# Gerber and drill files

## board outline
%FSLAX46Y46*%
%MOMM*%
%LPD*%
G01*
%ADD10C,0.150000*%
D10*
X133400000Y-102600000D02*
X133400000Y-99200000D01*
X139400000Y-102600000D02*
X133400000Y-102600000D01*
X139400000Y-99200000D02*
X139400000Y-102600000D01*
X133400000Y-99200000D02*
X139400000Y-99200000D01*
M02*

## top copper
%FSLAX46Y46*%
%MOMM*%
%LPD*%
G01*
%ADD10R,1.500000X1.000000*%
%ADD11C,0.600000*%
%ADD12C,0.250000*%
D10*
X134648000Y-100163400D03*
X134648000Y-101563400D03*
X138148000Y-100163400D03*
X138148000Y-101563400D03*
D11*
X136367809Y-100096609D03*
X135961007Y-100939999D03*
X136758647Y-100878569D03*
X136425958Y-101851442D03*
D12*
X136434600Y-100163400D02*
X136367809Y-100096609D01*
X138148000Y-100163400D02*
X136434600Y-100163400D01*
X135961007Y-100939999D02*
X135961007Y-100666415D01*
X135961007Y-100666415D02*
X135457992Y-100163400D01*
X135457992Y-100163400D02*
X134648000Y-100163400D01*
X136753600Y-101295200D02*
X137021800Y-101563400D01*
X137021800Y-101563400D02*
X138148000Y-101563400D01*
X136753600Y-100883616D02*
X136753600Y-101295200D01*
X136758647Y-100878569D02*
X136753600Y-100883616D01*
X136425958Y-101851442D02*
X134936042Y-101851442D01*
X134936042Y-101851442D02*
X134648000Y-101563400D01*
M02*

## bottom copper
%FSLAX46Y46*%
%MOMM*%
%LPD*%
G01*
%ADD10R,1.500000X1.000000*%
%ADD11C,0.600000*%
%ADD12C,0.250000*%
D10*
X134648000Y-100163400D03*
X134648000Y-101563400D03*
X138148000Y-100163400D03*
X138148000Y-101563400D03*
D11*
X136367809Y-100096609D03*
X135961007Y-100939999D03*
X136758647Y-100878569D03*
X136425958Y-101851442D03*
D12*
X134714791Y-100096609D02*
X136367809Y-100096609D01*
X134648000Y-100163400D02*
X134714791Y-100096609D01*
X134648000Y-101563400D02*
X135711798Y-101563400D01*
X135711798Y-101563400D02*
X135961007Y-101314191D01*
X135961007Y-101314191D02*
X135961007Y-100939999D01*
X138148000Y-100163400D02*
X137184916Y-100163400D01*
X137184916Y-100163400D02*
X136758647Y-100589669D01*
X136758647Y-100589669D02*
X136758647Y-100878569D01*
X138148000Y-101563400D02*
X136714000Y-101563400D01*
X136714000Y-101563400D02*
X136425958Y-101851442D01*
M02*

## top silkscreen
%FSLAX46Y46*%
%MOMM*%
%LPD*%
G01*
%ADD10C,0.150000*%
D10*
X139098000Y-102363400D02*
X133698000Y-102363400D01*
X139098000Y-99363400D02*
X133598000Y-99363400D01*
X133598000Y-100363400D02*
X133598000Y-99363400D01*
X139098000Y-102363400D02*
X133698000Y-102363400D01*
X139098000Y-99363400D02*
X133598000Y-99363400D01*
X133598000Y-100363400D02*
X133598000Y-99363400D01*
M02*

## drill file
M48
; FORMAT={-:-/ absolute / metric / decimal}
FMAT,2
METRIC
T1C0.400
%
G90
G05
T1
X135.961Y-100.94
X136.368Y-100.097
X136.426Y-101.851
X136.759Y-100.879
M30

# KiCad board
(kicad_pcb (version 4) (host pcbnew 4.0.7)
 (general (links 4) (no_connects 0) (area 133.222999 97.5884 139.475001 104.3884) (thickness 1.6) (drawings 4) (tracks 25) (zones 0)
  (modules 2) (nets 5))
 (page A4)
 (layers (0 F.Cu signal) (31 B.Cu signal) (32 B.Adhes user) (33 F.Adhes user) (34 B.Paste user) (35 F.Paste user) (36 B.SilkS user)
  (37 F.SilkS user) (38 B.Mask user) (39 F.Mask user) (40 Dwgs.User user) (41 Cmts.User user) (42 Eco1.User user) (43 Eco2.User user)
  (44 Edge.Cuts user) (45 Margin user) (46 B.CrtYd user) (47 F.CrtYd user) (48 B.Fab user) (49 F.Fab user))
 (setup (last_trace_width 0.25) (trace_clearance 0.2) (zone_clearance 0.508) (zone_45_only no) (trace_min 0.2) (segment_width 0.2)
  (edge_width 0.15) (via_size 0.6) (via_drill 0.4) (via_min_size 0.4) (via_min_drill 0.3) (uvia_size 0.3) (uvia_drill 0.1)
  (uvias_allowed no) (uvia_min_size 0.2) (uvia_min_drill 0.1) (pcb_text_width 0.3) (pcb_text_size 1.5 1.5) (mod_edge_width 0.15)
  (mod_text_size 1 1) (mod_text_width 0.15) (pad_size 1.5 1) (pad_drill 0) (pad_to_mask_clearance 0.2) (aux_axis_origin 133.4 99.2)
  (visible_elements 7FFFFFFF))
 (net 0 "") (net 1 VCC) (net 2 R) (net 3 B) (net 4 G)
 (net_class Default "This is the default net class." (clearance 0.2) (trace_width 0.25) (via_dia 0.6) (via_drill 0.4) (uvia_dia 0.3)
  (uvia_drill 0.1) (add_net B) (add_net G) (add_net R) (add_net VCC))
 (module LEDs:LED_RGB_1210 (layer F.Cu) (at 136.398 100.8634)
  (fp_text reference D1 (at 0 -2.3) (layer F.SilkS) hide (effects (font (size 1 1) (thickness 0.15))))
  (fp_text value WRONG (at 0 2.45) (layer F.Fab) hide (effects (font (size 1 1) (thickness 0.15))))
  (fp_line (start 2.7 1.5) (end -2.7 1.5) (layer F.SilkS) (width 0.15))
  (fp_line (start 2.7 -1.5) (end -2.8 -1.5) (layer F.SilkS) (width 0.15))
  (fp_line (start -2.8 -0.5) (end -2.8 -1.5) (layer F.SilkS) (width 0.15))
  (pad 1 smd rect (at -1.75 -0.7 180) (size 1.5 1) (layers B.Cu B.Paste B.Mask) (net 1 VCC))
  (pad 2 smd rect (at -1.75 0.7 180) (size 1.5 1) (layers B.Cu B.Paste B.Mask) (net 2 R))
  (pad 4 smd rect (at 1.75 -0.7 180) (size 1.5 1) (layers B.Cu B.Paste B.Mask) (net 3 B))
  (pad 3 smd rect (at 1.75 0.7 180) (size 1.5 1) (layers B.Cu B.Paste B.Mask) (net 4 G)))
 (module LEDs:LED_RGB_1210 (layer F.Cu) (at 136.398 100.8634)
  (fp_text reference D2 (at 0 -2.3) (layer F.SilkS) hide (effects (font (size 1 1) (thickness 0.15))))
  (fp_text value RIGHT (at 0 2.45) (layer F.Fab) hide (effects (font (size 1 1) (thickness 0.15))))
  (fp_line (start 2.7 1.5) (end -2.7 1.5) (layer F.SilkS) (width 0.15))
  (fp_line (start 2.7 -1.5) (end -2.8 -1.5) (layer F.SilkS) (width 0.15))
  (fp_line (start -2.8 -0.5) (end -2.8 -1.5) (layer F.SilkS) (width 0.15))
  (pad 1 smd rect (at -1.75 -0.7 180) (size 1.5 1) (layers F.Cu F.Paste F.Mask) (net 2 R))
  (pad 2 smd rect (at -1.75 0.7 180) (size 1.5 1) (layers F.Cu F.Paste F.Mask) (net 4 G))
  (pad 4 smd rect (at 1.75 -0.7 180) (size 1.5 1) (layers F.Cu F.Paste F.Mask) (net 1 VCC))
  (pad 3 smd rect (at 1.75 0.7 180) (size 1.5 1) (layers F.Cu F.Paste F.Mask) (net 3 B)))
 (gr_line (start 133.4 102.6) (end 133.4 99.2) (layer Edge.Cuts) (width 0.15))
 (gr_line (start 139.4 102.6) (end 133.4 102.6) (layer Edge.Cuts) (width 0.15))
 (gr_line (start 139.4 99.2) (end 139.4 102.6) (layer Edge.Cuts) (width 0.15))
 (gr_line (start 133.4 99.2) (end 139.4 99.2) (layer Edge.Cuts) (width 0.15))
 (segment (start 136.4346 100.1634) (end 136.367809 100.096609) (width 0.25) (layer F.Cu) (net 1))
 (segment (start 134.714791 100.096609) (end 136.367809 100.096609) (width 0.25) (layer B.Cu) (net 1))
 (segment (start 138.148 100.1634) (end 136.4346 100.1634) (width 0.25) (layer F.Cu) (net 1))
 (segment (start 134.648 100.1634) (end 134.714791 100.096609) (width 0.25) (layer B.Cu) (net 1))
 (via (at 136.367809 100.096609) (size 0.6) (drill 0.4) (layers F.Cu B.Cu) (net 1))
 (segment (start 134.648 101.5634) (end 135.711798 101.5634) (width 0.25) (layer B.Cu) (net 2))
 (segment (start 135.711798 101.5634) (end 135.961007 101.314191) (width 0.25) (layer B.Cu) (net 2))
 (segment (start 135.961007 101.314191) (end 135.961007 100.939999) (width 0.25) (layer B.Cu) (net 2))
 (segment (start 135.961007 100.939999) (end 135.961007 100.666415) (width 0.25) (layer F.Cu) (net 2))
 (segment (start 135.961007 100.666415) (end 135.457992 100.1634) (width 0.25) (layer F.Cu) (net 2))
 (segment (start 135.457992 100.1634) (end 134.648 100.1634) (width 0.25) (layer F.Cu) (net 2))
 (via (at 135.961007 100.939999) (size 0.6) (drill 0.4) (layers F.Cu B.Cu) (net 2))
 (segment (start 138.148 100.1634) (end 137.184916 100.1634) (width 0.25) (layer B.Cu) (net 3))
 (segment (start 137.184916 100.1634) (end 136.758647 100.589669) (width 0.25) (layer B.Cu) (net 3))
 (segment (start 136.758647 100.589669) (end 136.758647 100.878569) (width 0.25) (layer B.Cu) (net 3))
 (segment (start 136.7536 101.2952) (end 137.0218 101.5634) (width 0.25) (layer F.Cu) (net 3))
 (segment (start 137.0218 101.5634) (end 138.148 101.5634) (width 0.25) (layer F.Cu) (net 3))
 (segment (start 136.7536 100.883616) (end 136.7536 101.2952) (width 0.25) (layer F.Cu) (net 3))
 (segment (start 136.758647 100.878569) (end 136.7536 100.883616) (width 0.25) (layer F.Cu) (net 3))
 (via (at 136.758647 100.878569) (size 0.6) (drill 0.4) (layers F.Cu B.Cu) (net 3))
 (segment (start 136.425958 101.851442) (end 134.936042 101.851442) (width 0.25) (layer F.Cu) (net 4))
 (segment (start 134.936042 101.851442) (end 134.648 101.5634) (width 0.25) (layer F.Cu) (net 4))
 (segment (start 138.148 101.5634) (end 136.714 101.5634) (width 0.25) (layer B.Cu) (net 4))
 (segment (start 136.714 101.5634) (end 136.425958 101.851442) (width 0.25) (layer B.Cu) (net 4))
 (via (at 136.425958 101.851442) (size 0.6) (drill 0.4) (layers F.Cu B.Cu) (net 4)))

